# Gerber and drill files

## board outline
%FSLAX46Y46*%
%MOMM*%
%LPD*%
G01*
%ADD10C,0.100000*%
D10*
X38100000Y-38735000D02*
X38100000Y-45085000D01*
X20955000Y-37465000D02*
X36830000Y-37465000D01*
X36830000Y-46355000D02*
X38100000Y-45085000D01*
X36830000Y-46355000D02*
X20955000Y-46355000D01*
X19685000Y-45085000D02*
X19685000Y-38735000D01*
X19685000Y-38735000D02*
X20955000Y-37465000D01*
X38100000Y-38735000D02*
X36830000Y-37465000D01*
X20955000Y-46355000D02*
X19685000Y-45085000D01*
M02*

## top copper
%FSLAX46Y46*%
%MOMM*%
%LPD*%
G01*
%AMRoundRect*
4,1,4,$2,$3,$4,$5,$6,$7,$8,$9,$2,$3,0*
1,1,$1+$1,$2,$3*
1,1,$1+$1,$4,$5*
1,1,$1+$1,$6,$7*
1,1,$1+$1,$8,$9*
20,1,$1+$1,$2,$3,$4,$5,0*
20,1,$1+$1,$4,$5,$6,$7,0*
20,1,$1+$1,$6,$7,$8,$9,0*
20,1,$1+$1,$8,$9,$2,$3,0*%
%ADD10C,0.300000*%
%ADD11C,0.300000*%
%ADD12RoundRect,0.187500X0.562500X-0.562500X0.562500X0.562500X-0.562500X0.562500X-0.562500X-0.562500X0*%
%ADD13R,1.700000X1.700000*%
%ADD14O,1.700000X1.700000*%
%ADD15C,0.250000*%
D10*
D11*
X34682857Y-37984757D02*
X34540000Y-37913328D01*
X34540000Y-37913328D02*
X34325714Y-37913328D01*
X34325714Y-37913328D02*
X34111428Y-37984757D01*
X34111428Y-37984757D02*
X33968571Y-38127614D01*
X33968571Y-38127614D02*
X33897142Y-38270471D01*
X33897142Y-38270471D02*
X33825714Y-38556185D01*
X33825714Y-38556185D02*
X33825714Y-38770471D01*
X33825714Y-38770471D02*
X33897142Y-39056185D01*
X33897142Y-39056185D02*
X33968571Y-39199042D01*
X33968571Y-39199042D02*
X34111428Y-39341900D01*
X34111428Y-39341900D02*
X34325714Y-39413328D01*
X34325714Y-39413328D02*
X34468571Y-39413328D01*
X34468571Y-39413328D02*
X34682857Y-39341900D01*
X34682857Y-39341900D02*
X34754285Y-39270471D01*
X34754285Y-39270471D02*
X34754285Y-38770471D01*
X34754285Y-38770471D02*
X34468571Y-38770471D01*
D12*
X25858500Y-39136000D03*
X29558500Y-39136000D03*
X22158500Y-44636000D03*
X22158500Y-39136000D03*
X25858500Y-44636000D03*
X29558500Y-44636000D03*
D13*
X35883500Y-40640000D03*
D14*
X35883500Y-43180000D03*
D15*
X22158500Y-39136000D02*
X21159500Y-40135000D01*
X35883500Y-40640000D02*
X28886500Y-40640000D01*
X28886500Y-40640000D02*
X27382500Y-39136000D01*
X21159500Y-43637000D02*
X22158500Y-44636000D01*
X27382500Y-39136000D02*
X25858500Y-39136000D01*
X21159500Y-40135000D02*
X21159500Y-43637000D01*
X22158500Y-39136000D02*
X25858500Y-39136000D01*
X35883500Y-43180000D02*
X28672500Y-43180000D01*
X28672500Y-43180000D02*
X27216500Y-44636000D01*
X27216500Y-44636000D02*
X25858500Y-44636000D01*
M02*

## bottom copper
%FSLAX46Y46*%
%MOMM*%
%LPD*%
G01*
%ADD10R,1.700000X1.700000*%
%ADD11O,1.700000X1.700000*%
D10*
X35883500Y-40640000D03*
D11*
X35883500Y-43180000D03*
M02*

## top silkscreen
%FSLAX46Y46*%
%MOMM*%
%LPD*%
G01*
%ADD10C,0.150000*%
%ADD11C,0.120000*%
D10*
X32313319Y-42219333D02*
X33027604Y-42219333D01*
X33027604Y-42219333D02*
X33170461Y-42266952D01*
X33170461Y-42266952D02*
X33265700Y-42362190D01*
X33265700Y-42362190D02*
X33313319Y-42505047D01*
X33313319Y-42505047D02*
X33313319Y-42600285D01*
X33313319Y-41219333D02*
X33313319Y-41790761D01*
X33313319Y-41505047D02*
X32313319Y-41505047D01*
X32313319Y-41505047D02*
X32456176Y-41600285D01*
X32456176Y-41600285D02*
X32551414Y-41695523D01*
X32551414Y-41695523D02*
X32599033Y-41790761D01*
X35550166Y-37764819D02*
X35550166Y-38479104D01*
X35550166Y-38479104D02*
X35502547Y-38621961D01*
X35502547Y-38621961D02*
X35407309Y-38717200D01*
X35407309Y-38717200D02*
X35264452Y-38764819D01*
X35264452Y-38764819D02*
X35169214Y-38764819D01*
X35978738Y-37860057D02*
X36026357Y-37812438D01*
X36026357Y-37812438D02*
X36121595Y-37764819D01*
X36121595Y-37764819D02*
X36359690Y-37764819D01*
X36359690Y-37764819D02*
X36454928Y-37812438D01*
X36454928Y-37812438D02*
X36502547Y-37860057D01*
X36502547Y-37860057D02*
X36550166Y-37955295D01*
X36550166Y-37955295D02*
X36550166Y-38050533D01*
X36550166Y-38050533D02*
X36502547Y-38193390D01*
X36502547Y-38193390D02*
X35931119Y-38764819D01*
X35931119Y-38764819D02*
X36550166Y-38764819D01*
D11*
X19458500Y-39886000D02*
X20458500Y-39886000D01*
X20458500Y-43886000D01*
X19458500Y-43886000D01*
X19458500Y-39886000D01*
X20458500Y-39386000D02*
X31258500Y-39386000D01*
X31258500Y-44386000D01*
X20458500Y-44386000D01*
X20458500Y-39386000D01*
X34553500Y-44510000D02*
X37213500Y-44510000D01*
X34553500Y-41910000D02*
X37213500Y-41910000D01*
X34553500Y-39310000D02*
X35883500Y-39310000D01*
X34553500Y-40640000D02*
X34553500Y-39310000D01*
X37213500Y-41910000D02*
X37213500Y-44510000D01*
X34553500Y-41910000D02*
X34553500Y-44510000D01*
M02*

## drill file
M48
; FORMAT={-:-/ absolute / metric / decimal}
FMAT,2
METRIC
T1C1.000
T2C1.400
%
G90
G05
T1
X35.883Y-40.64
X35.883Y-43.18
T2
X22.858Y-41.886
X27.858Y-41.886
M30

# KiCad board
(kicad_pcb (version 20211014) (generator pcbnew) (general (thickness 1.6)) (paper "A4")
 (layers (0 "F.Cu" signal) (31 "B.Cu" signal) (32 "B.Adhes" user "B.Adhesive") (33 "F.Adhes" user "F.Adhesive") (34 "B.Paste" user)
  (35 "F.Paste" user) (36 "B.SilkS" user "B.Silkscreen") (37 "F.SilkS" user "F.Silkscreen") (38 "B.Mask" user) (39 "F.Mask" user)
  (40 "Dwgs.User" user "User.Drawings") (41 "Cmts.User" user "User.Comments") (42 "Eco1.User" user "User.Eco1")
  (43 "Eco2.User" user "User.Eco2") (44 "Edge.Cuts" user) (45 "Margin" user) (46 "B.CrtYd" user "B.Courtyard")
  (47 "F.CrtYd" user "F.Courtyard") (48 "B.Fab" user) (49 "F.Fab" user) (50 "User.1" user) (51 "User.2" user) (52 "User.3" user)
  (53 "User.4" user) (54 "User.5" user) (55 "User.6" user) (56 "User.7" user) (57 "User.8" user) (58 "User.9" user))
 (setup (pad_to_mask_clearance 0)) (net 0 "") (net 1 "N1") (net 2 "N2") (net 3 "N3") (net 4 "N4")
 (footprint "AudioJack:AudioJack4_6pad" (layer "F.Cu") (at 25.8585 41.886 90)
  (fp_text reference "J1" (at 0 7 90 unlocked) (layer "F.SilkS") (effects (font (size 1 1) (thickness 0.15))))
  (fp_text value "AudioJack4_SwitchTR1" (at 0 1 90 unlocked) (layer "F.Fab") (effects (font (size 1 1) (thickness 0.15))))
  (fp_rect (start -2 -5.4) (end 2 -6.4) (layer "F.SilkS") (width 0.12) (fill none))
  (fp_rect (start -2.5 -5.4) (end 2.5 5.4) (layer "F.SilkS") (width 0.12) (fill none))
  (pad "" np_thru_hole circle (at 0 2 90) (size 1.4 1.4) (drill 1.4) (layers F&B.Cu *.Mask))
  (pad "" np_thru_hole circle (at 0 -3 90) (size 1.4 1.4) (drill 1.4) (layers F&B.Cu *.Mask))
  (pad "R1" smd roundrect (at 2.75 0 90) (size 1.5 1.5) (layers "F.Cu" "F.Paste" "F.Mask") (roundrect_rratio 0.125) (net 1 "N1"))
  (pad "R1N" smd roundrect (at 2.75 3.7 90) (size 1.5 1.5) (layers "F.Cu" "F.Paste" "F.Mask") (roundrect_rratio 0.125) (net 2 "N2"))
  (pad "R2" smd roundrect (at -2.75 -3.7 90) (size 1.5 1.5) (layers "F.Cu" "F.Paste" "F.Mask") (roundrect_rratio 0.125) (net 1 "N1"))
  (pad "S" smd roundrect (at 2.75 -3.7 90) (size 1.5 1.5) (layers "F.Cu" "F.Paste" "F.Mask") (roundrect_rratio 0.125) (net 1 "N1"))
  (pad "T" smd roundrect (at -2.75 0 90) (size 1.5 1.5) (layers "F.Cu" "F.Paste" "F.Mask") (roundrect_rratio 0.125) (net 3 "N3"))
  (pad "TN" smd roundrect (at -2.75 3.7 90) (size 1.5 1.5) (layers "F.Cu" "F.Paste" "F.Mask") (roundrect_rratio 0.125) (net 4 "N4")))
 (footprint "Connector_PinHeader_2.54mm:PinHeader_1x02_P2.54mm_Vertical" (layer "F.Cu") (at 35.8835 40.64)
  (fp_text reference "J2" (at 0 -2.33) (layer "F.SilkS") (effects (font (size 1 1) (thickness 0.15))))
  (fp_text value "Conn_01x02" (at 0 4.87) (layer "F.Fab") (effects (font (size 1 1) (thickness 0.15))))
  (fp_line (start -1.33 3.87) (end 1.33 3.87) (layer "F.SilkS") (width 0.12))
  (fp_line (start -1.33 1.27) (end 1.33 1.27) (layer "F.SilkS") (width 0.12))
  (fp_line (start -1.33 -1.33) (end 0 -1.33) (layer "F.SilkS") (width 0.12))
  (fp_line (start -1.33 0) (end -1.33 -1.33) (layer "F.SilkS") (width 0.12))
  (fp_line (start 1.33 1.27) (end 1.33 3.87) (layer "F.SilkS") (width 0.12))
  (fp_line (start -1.33 1.27) (end -1.33 3.87) (layer "F.SilkS") (width 0.12))
  (pad "1" thru_hole rect locked (at 0 0) (size 1.7 1.7) (drill 1) (layers *.Cu *.Mask) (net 1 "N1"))
  (pad "2" thru_hole oval locked (at 0 2.54) (size 1.7 1.7) (drill 1) (layers *.Cu *.Mask) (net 3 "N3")))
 (gr_line (start 38.1 38.735) (end 38.1 45.085) (layer "Edge.Cuts") (width 0.1))
 (gr_line (start 20.955 37.465) (end 36.83 37.465) (layer "Edge.Cuts") (width 0.1))
 (gr_line (start 36.83 46.355) (end 38.1 45.085) (layer "Edge.Cuts") (width 0.1))
 (gr_line (start 36.83 46.355) (end 20.955 46.355) (layer "Edge.Cuts") (width 0.1))
 (gr_line (start 19.685 45.085) (end 19.685 38.735) (layer "Edge.Cuts") (width 0.1))
 (gr_line (start 19.685 38.735) (end 20.955 37.465) (layer "Edge.Cuts") (width 0.1))
 (gr_line (start 38.1 38.735) (end 36.83 37.465) (layer "Edge.Cuts") (width 0.1))
 (gr_line (start 20.955 46.355) (end 19.685 45.085) (layer "Edge.Cuts") (width 0.1))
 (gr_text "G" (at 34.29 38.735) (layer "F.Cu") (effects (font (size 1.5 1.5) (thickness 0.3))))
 (segment (start 22.1585 39.136) (end 21.1595 40.135) (width 0.25) (layer "F.Cu") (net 1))
 (segment (start 35.8835 40.64) (end 28.8865 40.64) (width 0.25) (layer "F.Cu") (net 1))
 (segment (start 28.8865 40.64) (end 27.3825 39.136) (width 0.25) (layer "F.Cu") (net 1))
 (segment (start 21.1595 43.637) (end 22.1585 44.636) (width 0.25) (layer "F.Cu") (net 1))
 (segment (start 27.3825 39.136) (end 25.8585 39.136) (width 0.25) (layer "F.Cu") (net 1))
 (segment (start 21.1595 40.135) (end 21.1595 43.637) (width 0.25) (layer "F.Cu") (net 1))
 (segment (start 22.1585 39.136) (end 25.8585 39.136) (width 0.25) (layer "F.Cu") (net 1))
 (segment (start 35.8835 43.18) (end 28.6725 43.18) (width 0.25) (layer "F.Cu") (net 3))
 (segment (start 28.6725 43.18) (end 27.2165 44.636) (width 0.25) (layer "F.Cu") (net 3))
 (segment (start 27.2165 44.636) (end 25.8585 44.636) (width 0.25) (layer "F.Cu") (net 3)))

